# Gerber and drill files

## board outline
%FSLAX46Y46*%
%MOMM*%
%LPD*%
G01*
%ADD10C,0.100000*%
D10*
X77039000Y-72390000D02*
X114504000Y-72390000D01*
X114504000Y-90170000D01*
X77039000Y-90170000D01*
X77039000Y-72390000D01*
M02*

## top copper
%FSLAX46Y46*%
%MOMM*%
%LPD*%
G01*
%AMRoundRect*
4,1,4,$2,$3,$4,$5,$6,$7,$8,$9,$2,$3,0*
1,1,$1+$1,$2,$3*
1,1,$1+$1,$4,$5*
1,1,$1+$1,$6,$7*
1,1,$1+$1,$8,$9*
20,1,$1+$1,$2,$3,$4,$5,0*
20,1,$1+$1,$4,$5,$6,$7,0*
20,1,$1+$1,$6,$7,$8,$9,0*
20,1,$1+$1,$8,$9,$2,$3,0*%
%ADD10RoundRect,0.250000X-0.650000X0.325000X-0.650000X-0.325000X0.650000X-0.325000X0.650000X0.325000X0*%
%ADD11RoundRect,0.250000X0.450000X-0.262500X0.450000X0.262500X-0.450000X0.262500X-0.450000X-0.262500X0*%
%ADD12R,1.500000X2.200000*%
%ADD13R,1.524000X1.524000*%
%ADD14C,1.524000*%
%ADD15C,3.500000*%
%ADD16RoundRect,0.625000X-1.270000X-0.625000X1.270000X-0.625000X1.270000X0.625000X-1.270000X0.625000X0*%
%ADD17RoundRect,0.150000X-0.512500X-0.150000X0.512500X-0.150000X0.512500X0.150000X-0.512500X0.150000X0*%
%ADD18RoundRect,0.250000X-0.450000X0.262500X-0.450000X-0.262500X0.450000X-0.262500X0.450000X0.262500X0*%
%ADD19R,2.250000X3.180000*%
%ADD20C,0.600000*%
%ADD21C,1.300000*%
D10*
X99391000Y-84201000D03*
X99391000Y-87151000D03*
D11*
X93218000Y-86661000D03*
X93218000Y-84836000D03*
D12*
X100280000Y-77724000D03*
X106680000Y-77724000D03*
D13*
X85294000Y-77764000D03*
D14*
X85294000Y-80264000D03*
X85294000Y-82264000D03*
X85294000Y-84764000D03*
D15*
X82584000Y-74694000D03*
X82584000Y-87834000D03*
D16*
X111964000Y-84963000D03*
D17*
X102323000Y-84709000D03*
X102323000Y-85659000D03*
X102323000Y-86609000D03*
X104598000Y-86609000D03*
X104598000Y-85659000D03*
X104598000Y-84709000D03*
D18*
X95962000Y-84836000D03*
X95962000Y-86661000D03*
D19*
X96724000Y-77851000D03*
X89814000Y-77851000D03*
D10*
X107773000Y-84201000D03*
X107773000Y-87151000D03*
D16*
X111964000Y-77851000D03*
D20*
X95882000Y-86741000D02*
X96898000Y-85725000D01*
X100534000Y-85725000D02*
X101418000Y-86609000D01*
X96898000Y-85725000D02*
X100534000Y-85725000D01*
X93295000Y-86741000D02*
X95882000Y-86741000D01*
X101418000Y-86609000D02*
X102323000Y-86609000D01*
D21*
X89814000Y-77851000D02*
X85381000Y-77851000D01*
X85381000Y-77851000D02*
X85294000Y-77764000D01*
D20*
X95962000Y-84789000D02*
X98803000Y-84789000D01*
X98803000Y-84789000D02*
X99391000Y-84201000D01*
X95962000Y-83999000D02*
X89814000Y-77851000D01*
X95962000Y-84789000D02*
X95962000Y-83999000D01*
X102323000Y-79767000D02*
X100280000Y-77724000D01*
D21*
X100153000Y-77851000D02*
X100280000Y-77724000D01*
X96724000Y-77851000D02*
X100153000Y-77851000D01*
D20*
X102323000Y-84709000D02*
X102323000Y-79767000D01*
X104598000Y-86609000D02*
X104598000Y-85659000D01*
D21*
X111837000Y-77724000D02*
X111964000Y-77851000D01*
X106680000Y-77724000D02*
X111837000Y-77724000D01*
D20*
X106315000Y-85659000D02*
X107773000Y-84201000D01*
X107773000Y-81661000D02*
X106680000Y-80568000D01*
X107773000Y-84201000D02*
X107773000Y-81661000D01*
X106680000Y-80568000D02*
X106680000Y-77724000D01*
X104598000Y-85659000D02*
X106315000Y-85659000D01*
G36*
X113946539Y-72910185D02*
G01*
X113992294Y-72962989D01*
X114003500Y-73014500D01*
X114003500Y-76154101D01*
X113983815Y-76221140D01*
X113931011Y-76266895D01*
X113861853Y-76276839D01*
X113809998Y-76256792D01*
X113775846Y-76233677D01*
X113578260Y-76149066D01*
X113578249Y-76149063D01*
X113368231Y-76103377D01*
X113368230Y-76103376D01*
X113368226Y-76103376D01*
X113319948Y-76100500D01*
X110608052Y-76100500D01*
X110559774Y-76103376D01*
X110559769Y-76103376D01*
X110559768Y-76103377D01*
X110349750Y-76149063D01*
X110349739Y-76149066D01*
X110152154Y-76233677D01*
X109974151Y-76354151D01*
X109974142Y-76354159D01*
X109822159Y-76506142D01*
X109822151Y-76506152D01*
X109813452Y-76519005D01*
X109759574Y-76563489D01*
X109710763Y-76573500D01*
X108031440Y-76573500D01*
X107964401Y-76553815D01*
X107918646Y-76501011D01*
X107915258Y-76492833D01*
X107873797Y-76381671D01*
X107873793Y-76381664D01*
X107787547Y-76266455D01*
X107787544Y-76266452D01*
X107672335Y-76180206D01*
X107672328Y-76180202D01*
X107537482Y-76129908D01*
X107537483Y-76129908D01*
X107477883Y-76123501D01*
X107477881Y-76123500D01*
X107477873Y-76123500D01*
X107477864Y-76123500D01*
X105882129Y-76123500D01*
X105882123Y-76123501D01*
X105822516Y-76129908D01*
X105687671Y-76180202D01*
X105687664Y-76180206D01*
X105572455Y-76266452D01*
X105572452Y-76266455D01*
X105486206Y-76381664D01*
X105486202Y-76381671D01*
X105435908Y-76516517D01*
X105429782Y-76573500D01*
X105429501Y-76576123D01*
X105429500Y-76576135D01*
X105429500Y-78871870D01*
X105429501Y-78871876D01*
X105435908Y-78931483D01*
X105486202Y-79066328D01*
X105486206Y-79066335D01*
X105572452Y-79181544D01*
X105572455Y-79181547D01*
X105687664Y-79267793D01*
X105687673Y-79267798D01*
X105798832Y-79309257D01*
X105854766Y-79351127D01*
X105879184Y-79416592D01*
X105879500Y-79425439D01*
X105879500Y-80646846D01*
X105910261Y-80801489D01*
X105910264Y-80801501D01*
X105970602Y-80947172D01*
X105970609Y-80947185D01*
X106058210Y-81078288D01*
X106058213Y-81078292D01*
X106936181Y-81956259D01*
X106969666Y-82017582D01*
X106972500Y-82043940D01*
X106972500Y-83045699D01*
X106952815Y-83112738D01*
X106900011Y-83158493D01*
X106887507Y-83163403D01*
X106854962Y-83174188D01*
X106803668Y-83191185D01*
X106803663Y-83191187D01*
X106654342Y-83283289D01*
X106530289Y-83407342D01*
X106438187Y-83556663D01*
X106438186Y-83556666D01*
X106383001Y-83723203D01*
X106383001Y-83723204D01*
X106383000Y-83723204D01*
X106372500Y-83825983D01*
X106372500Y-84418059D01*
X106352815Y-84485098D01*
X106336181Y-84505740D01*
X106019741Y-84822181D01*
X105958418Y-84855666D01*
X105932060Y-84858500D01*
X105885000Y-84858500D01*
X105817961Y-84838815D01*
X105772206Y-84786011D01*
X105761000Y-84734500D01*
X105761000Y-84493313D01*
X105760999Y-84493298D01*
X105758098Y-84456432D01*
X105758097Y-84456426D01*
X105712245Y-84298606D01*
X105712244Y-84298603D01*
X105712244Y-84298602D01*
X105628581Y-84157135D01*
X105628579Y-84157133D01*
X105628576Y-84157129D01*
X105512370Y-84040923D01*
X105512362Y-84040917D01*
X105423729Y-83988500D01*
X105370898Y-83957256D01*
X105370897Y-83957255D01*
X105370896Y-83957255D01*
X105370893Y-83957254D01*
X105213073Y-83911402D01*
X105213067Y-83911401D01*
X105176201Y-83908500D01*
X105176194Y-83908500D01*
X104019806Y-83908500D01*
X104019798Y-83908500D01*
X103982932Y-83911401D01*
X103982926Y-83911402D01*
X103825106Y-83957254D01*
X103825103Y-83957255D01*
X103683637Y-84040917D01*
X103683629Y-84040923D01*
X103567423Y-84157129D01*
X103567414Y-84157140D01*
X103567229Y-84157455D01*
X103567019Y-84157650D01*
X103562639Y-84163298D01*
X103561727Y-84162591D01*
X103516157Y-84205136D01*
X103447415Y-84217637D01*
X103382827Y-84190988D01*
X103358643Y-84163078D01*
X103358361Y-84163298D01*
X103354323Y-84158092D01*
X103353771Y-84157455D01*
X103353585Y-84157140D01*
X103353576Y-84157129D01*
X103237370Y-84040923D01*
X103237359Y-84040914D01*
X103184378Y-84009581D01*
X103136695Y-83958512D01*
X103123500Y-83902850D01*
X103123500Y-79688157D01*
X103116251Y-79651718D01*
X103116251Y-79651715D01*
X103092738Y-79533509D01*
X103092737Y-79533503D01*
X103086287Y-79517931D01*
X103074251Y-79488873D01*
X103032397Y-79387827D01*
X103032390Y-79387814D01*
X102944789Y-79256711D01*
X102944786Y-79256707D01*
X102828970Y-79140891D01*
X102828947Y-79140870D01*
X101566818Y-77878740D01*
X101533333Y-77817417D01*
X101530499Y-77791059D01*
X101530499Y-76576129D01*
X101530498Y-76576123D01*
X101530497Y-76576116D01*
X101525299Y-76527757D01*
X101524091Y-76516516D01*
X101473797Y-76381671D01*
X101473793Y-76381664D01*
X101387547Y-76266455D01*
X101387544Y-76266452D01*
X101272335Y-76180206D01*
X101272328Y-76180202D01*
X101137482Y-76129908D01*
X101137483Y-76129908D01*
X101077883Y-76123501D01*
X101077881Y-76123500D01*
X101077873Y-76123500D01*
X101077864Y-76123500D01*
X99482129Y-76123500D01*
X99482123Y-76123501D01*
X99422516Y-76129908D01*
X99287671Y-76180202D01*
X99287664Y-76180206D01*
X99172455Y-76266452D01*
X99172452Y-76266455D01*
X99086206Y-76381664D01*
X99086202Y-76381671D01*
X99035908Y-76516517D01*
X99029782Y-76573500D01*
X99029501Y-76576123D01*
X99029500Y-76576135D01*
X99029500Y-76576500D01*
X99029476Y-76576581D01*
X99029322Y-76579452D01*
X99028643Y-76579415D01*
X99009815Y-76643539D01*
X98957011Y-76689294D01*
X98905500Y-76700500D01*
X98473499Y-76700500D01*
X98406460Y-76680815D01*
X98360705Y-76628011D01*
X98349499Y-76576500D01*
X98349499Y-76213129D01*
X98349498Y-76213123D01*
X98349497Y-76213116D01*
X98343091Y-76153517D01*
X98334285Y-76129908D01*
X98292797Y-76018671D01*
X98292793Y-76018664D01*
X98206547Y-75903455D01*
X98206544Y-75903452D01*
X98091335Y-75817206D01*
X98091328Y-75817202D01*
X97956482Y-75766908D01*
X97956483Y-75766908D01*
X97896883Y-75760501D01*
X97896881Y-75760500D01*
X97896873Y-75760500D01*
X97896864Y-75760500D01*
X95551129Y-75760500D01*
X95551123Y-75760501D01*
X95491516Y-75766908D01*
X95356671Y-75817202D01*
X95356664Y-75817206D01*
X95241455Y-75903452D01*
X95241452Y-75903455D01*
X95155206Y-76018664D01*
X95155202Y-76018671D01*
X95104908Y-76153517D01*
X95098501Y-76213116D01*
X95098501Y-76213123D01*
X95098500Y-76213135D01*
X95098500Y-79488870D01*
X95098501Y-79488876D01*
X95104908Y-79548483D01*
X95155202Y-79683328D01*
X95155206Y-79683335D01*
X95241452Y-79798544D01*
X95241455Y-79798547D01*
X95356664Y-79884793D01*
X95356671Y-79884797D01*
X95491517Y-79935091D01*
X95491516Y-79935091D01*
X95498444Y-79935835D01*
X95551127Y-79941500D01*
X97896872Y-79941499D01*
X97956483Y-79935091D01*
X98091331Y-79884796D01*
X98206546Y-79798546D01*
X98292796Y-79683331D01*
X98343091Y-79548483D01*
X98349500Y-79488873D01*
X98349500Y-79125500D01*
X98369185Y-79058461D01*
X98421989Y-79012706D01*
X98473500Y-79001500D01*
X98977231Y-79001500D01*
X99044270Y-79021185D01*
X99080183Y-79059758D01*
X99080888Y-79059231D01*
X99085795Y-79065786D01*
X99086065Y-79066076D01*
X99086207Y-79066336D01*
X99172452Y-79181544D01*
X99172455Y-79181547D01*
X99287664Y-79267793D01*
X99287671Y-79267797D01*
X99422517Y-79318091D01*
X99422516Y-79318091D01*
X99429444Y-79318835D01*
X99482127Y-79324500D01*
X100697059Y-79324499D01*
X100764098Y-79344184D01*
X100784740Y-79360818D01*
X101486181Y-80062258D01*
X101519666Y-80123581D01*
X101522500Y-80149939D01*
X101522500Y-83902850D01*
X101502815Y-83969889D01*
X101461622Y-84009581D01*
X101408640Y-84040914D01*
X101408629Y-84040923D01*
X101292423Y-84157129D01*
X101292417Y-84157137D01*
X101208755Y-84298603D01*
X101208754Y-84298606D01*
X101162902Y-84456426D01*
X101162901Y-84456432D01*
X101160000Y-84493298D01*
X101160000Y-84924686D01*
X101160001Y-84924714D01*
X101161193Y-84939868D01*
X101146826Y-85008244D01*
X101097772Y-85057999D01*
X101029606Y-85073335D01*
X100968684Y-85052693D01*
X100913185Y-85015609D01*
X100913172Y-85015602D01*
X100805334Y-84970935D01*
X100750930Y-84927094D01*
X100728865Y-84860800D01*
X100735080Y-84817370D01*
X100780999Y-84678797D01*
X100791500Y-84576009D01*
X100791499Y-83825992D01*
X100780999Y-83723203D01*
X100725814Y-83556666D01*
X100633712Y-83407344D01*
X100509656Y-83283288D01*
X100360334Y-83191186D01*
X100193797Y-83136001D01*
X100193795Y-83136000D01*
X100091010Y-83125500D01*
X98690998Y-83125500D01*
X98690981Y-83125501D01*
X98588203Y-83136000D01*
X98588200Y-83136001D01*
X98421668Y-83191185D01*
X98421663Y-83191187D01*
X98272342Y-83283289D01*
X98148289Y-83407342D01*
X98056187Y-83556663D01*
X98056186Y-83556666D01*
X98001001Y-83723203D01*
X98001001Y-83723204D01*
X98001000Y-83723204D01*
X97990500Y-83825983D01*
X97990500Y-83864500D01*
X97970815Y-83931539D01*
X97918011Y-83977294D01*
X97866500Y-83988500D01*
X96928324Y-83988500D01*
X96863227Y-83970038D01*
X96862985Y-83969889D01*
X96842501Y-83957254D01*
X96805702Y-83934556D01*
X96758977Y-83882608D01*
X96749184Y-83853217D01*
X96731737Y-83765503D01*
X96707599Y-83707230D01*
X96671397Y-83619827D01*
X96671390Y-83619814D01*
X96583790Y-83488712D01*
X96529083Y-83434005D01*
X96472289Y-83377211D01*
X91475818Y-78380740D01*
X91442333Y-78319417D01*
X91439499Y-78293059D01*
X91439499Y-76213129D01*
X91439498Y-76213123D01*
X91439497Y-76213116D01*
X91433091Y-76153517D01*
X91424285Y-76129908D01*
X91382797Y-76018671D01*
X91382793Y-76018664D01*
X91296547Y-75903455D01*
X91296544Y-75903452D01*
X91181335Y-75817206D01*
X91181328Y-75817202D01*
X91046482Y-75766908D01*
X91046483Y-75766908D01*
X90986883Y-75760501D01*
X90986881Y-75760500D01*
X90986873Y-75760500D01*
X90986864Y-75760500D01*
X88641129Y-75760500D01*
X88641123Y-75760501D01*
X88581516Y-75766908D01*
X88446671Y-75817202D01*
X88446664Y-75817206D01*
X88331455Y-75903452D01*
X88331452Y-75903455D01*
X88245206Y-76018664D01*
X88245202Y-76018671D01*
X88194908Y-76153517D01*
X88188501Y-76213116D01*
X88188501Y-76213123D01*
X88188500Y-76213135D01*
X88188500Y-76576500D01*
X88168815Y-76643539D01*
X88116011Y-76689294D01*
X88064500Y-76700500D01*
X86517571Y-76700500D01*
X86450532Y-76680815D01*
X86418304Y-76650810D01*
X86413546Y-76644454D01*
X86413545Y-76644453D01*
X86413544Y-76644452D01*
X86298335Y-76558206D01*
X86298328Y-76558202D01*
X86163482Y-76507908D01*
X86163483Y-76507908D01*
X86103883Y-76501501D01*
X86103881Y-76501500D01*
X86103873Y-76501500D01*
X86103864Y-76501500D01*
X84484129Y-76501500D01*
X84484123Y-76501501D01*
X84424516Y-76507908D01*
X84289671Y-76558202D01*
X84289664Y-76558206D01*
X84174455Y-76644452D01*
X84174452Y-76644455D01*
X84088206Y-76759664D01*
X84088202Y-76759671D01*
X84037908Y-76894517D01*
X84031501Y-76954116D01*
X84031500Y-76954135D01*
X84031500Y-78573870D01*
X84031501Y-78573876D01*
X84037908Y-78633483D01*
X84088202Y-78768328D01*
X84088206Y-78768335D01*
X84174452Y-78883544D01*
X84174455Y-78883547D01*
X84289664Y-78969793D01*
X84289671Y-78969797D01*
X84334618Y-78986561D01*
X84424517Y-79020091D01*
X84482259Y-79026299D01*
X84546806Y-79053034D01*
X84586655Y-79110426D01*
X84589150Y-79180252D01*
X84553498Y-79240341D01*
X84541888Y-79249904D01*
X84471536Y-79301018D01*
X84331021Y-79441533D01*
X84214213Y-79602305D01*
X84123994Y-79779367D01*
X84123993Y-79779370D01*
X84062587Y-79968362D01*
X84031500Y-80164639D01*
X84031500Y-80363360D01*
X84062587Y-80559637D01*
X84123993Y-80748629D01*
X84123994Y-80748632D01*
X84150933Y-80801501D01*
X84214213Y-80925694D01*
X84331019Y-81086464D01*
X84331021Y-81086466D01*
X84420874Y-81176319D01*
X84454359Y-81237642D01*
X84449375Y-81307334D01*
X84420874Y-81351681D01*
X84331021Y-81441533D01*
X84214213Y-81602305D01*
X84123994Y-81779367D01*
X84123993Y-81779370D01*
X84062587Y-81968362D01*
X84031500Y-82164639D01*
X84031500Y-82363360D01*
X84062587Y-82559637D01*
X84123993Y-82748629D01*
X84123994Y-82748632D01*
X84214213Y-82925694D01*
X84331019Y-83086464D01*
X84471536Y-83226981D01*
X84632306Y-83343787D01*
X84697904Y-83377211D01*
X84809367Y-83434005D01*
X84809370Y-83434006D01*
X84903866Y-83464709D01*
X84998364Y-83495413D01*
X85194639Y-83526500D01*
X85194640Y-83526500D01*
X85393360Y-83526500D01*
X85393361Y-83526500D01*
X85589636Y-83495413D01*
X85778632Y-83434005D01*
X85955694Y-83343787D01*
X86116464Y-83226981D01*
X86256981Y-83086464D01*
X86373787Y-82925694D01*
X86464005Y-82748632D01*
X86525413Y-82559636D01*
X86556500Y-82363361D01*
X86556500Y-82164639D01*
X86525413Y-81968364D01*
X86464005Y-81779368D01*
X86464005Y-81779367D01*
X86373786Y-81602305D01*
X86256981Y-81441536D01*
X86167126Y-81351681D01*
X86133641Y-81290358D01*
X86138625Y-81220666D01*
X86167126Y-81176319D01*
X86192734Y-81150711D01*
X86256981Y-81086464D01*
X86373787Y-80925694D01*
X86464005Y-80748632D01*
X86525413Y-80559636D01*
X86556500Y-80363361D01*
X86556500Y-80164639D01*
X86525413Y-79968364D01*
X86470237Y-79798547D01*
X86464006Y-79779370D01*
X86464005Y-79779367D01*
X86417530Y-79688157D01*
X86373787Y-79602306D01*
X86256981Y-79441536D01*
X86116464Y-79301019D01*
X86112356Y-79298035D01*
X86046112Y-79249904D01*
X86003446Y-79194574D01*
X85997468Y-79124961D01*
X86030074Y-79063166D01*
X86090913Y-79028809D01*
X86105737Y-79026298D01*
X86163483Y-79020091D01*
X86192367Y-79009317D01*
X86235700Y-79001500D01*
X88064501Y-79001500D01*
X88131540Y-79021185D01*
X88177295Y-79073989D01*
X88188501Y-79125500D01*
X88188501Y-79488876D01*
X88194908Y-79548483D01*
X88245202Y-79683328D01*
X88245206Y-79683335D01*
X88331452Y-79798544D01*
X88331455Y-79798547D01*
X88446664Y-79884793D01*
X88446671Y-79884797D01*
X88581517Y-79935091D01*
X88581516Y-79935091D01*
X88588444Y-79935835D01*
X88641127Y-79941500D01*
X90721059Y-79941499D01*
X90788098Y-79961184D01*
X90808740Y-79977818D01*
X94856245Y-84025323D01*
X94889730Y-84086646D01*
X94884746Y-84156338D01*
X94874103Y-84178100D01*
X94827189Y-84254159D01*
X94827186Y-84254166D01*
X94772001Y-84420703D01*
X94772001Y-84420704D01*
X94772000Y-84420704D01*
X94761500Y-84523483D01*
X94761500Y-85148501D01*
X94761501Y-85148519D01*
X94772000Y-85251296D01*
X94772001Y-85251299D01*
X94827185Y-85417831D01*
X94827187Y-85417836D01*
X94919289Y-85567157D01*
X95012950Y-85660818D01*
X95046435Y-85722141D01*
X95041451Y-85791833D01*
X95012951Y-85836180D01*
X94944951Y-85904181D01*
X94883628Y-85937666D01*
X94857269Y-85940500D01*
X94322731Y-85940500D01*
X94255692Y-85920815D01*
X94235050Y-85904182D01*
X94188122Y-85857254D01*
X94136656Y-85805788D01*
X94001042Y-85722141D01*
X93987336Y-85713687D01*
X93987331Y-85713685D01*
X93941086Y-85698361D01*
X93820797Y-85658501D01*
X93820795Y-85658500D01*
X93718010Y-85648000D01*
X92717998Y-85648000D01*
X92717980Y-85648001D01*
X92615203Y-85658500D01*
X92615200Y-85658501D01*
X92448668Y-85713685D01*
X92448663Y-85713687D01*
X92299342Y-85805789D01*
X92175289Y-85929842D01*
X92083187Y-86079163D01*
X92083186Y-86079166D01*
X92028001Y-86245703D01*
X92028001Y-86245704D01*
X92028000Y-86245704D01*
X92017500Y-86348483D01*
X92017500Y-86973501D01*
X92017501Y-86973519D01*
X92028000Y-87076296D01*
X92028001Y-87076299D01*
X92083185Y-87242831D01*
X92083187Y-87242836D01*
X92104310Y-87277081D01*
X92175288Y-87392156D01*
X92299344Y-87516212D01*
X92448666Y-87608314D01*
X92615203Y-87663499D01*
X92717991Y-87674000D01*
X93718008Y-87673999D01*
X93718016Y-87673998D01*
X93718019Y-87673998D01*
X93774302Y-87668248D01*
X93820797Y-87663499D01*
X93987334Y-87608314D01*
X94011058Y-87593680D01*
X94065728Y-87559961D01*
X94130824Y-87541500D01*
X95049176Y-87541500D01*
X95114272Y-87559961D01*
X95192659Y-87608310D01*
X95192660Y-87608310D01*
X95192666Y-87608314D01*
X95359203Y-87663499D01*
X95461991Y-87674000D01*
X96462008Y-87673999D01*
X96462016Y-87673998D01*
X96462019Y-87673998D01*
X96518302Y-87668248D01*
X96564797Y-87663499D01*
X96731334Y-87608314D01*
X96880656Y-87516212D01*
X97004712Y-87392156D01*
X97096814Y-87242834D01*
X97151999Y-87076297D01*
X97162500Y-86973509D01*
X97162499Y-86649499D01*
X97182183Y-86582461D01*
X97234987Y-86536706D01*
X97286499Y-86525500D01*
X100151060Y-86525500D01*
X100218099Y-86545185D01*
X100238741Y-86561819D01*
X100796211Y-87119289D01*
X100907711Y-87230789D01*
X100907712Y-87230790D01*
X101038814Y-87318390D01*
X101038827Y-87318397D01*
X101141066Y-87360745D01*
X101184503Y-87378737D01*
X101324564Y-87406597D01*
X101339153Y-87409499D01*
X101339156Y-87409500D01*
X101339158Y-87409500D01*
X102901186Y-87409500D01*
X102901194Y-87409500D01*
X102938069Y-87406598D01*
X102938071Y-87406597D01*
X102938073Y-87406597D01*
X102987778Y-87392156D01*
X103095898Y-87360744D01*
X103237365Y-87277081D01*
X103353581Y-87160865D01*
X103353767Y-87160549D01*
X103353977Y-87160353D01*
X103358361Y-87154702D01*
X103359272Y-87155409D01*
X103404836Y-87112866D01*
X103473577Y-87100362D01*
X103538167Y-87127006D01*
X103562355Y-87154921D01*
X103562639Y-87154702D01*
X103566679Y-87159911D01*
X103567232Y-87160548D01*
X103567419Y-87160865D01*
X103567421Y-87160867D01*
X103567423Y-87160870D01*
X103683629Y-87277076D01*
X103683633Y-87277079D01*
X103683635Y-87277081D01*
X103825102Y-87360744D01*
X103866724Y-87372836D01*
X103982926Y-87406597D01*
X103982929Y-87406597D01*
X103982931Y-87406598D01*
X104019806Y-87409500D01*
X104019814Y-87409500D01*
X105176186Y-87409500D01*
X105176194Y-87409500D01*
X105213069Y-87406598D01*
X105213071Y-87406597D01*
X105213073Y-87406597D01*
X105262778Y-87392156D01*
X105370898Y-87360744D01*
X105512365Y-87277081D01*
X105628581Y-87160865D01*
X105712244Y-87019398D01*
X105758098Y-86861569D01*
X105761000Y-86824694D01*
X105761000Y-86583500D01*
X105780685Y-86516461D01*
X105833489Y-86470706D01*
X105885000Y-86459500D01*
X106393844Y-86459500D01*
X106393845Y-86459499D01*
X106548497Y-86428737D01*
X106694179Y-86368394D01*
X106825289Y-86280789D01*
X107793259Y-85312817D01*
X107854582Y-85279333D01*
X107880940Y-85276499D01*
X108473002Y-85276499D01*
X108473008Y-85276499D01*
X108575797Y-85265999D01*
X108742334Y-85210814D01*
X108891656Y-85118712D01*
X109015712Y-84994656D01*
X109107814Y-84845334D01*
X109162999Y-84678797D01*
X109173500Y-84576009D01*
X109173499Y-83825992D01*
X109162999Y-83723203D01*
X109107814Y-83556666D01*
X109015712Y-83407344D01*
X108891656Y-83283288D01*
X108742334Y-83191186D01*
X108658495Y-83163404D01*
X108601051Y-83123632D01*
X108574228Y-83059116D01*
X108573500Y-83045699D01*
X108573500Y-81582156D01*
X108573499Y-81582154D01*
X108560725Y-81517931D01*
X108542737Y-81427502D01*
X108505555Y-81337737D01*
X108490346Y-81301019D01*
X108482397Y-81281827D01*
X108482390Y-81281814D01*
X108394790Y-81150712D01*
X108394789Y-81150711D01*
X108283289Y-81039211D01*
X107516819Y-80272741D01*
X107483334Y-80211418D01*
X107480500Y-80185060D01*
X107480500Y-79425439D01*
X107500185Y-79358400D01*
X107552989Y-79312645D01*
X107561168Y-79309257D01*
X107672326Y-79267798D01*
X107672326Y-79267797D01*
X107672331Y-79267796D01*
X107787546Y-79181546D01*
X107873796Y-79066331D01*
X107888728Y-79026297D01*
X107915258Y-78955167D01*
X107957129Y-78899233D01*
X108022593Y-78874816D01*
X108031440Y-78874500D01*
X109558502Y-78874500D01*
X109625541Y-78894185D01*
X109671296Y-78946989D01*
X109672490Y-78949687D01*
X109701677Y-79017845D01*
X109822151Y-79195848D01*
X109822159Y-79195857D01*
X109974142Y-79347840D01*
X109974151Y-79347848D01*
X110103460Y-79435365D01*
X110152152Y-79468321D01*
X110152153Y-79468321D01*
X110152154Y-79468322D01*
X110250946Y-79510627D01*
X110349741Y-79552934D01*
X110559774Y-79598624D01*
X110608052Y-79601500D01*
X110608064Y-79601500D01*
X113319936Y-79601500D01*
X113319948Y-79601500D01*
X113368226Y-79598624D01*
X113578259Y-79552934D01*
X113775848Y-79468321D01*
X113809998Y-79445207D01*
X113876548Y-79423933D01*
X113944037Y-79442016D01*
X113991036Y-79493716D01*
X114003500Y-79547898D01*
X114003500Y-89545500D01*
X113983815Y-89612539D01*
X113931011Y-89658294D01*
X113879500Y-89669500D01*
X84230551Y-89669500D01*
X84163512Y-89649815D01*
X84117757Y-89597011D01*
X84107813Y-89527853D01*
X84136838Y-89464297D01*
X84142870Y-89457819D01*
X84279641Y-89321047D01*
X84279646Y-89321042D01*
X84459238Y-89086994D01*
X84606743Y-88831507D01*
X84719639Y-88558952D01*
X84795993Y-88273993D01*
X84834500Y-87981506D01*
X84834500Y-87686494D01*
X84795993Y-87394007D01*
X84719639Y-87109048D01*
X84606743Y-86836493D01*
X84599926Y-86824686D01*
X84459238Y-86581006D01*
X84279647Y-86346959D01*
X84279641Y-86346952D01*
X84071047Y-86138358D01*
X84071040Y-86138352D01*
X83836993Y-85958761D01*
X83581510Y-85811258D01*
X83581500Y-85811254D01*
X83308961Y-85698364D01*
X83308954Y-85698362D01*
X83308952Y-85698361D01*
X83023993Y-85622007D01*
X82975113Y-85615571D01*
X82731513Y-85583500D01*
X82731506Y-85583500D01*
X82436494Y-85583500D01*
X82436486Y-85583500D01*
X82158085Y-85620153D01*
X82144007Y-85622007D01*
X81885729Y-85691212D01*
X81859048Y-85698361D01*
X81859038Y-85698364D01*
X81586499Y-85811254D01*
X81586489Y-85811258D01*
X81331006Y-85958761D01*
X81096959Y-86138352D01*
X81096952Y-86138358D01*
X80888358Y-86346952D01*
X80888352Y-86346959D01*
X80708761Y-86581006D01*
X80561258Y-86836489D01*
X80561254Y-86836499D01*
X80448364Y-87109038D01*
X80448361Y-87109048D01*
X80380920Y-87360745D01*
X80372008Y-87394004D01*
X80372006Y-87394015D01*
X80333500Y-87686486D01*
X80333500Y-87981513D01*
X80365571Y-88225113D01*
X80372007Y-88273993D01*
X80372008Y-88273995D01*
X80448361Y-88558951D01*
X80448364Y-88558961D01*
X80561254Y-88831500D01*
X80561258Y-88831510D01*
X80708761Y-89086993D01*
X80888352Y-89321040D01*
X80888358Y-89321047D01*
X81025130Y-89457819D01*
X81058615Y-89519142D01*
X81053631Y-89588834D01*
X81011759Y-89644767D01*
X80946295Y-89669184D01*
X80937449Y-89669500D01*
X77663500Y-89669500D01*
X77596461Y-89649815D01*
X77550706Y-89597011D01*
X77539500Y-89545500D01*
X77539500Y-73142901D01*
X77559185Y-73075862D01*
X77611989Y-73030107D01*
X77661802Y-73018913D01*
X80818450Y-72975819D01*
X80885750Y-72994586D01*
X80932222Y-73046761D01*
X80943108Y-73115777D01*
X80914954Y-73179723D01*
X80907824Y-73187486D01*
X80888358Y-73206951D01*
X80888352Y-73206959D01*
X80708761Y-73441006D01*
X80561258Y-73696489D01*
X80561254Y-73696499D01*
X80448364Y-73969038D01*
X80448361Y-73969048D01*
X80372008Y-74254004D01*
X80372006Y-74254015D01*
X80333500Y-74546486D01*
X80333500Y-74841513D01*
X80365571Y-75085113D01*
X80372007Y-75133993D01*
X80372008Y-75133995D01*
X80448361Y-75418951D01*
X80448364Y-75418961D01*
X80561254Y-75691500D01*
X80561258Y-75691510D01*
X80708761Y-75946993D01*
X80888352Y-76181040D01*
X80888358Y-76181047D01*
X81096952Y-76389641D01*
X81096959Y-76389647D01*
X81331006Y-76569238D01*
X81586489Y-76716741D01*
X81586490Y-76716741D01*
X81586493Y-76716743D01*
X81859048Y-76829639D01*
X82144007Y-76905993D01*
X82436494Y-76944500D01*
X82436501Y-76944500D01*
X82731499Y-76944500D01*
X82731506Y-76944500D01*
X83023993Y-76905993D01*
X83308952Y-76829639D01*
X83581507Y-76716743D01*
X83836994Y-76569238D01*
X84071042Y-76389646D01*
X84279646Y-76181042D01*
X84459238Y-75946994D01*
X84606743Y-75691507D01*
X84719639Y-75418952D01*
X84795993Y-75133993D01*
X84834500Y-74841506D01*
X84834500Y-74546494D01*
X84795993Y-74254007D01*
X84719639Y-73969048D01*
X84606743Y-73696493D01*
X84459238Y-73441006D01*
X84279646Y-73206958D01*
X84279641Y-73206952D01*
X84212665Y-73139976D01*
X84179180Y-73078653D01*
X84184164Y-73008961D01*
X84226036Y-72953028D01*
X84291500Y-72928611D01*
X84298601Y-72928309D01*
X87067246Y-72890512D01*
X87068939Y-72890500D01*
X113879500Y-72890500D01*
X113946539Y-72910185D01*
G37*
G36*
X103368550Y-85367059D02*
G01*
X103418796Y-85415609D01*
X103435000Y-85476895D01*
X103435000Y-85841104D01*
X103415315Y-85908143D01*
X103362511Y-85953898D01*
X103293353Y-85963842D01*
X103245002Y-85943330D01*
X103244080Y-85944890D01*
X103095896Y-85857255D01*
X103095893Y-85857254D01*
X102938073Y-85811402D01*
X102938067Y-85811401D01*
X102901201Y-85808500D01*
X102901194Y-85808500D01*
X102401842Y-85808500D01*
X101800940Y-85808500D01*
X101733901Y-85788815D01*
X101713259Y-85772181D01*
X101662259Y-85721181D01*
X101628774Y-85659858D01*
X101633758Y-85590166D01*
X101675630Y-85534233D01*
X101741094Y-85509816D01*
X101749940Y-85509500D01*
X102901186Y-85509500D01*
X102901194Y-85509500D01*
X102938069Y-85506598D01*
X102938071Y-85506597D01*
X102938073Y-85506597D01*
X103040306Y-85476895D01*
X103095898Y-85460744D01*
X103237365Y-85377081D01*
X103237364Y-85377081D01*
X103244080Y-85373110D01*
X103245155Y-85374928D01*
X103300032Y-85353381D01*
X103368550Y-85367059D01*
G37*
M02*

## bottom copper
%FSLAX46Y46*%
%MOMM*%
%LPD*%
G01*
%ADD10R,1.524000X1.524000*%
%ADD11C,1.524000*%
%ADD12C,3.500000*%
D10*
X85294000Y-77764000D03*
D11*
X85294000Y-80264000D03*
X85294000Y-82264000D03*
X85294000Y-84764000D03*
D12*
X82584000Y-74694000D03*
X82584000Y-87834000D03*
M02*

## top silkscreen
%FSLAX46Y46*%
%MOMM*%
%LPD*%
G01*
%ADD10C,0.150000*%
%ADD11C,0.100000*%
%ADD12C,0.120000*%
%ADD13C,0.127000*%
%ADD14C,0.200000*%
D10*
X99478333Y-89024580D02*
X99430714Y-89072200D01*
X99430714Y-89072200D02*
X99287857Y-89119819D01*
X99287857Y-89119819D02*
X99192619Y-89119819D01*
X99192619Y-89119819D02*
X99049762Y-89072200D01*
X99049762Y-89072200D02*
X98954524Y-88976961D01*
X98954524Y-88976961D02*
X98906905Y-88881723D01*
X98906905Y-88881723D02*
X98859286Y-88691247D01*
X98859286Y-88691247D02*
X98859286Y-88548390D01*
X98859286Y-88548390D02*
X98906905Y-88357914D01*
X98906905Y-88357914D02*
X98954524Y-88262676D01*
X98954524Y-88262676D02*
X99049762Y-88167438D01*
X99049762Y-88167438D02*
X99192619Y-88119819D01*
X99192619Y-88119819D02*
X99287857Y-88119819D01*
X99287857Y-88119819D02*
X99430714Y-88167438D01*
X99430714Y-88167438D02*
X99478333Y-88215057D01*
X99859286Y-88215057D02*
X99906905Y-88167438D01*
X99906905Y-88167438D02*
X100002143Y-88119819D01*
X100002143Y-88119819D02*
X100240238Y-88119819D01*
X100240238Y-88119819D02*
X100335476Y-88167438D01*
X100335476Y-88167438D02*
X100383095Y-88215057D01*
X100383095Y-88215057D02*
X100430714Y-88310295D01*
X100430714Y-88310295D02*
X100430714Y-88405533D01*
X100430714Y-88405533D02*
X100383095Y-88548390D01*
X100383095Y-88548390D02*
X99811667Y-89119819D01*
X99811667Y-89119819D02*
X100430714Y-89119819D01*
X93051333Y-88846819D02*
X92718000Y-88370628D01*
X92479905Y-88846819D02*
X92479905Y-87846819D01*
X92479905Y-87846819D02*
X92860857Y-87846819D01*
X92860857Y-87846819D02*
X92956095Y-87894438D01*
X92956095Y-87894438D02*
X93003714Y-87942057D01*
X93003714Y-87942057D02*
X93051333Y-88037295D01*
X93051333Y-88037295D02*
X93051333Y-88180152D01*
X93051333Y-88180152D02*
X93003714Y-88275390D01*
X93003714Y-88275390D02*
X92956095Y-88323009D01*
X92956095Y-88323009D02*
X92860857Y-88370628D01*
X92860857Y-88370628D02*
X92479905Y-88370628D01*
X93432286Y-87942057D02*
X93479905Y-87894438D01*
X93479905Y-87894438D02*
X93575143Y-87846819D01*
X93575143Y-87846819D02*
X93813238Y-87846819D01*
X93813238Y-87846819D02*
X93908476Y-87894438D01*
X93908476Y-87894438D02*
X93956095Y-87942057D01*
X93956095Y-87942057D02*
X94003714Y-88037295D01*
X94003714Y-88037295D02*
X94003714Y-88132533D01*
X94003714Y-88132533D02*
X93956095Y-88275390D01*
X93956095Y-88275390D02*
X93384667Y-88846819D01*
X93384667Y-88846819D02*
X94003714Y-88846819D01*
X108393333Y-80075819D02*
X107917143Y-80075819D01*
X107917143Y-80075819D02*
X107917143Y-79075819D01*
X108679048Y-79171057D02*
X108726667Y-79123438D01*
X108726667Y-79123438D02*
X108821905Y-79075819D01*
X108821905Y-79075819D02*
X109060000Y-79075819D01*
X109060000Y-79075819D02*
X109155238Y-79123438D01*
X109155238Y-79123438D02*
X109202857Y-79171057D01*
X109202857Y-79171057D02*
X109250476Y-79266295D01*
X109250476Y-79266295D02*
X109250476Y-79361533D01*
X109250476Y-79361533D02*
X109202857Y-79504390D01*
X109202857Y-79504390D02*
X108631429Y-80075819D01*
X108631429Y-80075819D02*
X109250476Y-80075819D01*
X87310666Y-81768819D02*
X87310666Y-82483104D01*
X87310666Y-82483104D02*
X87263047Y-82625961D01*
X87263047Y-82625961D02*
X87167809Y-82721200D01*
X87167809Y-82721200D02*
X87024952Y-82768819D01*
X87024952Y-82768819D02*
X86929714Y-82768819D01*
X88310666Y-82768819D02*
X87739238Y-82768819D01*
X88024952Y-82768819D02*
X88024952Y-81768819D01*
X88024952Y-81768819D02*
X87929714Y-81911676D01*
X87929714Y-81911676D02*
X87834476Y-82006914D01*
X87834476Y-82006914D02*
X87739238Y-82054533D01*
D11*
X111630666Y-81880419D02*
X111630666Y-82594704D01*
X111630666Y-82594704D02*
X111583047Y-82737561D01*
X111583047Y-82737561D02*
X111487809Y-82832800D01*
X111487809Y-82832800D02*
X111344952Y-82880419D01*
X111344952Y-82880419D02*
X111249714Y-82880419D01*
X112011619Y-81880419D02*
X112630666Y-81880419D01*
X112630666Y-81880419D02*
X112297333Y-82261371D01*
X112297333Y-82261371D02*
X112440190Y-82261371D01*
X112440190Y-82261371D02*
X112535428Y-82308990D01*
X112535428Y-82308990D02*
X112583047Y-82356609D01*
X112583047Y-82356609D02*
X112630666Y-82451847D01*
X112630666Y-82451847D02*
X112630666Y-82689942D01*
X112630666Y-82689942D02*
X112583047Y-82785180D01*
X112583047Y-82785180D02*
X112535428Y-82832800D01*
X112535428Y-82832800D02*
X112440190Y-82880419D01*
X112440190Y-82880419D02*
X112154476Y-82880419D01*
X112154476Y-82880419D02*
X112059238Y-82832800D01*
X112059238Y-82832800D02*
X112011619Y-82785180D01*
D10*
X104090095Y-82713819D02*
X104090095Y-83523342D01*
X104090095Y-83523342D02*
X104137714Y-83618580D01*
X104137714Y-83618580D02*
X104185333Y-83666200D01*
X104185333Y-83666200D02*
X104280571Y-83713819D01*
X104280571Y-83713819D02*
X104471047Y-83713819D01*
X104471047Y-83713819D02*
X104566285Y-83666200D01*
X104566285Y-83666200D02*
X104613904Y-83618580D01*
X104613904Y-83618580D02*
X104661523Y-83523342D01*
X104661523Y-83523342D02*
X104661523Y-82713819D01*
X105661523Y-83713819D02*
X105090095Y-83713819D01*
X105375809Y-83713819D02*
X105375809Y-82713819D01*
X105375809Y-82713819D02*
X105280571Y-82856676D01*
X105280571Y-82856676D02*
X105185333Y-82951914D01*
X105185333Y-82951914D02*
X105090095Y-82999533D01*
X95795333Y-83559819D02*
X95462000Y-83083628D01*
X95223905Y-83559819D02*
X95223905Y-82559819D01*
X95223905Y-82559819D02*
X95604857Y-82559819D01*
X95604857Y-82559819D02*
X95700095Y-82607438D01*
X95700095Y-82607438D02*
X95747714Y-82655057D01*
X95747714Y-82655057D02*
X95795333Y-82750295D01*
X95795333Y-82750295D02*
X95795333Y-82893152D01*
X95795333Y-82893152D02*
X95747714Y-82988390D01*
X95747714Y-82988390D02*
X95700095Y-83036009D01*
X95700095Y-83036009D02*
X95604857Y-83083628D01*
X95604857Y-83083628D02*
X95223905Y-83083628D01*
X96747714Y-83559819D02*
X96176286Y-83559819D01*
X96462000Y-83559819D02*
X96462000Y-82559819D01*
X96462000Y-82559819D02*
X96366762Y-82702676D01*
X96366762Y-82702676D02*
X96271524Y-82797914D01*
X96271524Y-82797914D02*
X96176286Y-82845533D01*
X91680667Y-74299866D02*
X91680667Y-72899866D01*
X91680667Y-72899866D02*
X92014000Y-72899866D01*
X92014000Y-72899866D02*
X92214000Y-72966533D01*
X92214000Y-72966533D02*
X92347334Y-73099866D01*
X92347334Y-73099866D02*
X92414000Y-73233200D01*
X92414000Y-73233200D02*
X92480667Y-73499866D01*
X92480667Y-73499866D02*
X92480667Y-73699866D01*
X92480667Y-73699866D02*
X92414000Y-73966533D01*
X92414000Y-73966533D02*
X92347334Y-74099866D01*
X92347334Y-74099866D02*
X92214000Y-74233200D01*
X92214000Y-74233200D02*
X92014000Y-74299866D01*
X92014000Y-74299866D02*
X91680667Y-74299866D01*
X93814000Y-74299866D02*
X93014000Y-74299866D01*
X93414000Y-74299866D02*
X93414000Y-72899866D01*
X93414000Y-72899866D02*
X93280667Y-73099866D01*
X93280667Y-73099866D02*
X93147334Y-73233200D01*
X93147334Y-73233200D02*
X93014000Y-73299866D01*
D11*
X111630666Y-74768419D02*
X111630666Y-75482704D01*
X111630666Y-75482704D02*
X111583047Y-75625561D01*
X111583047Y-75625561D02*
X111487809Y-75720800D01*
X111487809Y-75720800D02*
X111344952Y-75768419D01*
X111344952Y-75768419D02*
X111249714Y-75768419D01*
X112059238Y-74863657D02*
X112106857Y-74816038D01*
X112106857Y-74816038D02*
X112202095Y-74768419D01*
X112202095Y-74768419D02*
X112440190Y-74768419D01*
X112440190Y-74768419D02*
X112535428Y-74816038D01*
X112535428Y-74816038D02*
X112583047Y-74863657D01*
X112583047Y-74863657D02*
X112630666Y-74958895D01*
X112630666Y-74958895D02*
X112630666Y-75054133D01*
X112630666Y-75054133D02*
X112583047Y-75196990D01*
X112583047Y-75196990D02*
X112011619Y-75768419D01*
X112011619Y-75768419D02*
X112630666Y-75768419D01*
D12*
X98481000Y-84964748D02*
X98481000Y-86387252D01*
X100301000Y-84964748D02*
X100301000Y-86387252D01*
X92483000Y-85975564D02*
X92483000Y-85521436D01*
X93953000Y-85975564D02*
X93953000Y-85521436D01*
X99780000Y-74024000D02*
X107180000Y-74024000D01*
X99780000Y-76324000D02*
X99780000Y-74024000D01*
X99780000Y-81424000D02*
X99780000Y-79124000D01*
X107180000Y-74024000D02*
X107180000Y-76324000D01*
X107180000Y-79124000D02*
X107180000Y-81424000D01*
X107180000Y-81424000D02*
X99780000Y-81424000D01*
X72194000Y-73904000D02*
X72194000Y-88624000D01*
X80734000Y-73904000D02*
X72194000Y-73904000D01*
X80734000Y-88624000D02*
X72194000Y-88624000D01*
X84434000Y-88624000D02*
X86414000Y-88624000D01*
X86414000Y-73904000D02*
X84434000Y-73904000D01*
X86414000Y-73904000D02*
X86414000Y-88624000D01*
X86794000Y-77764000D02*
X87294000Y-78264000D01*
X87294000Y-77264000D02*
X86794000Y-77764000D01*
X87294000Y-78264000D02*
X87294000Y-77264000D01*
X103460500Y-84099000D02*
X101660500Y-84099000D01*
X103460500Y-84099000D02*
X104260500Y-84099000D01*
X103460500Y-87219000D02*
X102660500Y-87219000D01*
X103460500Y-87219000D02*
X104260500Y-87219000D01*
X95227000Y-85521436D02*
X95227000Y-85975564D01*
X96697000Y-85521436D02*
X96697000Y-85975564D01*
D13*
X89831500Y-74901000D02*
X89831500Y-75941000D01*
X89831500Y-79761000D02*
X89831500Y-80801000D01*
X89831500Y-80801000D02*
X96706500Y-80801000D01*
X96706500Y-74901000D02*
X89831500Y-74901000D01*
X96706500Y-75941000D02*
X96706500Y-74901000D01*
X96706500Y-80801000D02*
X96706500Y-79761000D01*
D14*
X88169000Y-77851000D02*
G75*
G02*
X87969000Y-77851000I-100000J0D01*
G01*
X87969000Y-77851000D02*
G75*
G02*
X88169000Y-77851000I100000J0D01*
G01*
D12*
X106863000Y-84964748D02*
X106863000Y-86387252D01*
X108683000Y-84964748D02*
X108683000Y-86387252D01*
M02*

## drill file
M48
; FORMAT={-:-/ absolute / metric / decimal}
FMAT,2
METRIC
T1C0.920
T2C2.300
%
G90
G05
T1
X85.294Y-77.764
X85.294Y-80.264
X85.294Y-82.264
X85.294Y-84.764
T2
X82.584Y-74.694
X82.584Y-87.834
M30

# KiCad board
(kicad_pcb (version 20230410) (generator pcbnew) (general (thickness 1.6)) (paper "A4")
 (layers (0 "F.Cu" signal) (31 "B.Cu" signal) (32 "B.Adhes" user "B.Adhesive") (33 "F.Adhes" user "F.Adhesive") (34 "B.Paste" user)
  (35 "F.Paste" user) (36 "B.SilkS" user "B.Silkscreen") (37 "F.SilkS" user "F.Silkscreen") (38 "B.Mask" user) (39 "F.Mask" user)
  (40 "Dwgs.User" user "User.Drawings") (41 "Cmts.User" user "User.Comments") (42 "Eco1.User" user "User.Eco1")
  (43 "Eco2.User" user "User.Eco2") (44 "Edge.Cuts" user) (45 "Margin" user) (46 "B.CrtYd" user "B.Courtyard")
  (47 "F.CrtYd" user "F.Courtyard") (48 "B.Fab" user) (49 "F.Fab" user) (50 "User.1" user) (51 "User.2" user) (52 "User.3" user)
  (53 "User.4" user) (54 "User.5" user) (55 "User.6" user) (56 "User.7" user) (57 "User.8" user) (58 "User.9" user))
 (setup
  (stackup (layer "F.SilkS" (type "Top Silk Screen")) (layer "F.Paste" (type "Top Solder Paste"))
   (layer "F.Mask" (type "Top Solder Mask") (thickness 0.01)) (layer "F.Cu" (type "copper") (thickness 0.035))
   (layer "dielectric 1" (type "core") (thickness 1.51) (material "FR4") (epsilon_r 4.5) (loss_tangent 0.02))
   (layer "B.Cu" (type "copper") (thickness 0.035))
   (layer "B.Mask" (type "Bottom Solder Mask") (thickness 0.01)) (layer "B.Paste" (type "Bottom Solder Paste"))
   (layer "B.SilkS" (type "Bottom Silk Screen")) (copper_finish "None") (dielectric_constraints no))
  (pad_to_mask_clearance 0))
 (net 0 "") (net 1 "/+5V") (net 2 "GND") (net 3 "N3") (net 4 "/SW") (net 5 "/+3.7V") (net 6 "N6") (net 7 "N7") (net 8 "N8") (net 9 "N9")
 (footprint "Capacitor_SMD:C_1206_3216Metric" (layer "F.Cu") (at 99.391 85.676 -90)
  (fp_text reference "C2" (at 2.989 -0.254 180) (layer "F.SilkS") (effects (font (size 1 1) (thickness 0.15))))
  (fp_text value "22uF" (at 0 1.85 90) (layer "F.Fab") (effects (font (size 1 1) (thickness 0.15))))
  (fp_line (start -0.711252 0.91) (end 0.711252 0.91) (stroke (width 0.12) (type solid)) (layer "F.SilkS"))
  (fp_line (start -0.711252 -0.91) (end 0.711252 -0.91) (stroke (width 0.12) (type solid)) (layer "F.SilkS"))
  (pad "1" smd roundrect (at -1.475 0 270) (size 1.15 1.8) (layers "F.Cu" "F.Paste" "F.Mask") (roundrect_rratio 0.217391) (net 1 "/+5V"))
  (pad "2" smd roundrect (at 1.475 0 270) (size 1.15 1.8) (layers "F.Cu" "F.Paste" "F.Mask") (roundrect_rratio 0.217391) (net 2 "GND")))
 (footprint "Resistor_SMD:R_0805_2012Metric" (layer "F.Cu") (at 93.218 85.7485 90)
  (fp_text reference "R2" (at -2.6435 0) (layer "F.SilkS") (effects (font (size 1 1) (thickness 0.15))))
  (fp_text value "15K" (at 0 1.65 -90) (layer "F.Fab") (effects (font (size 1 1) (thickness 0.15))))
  (fp_line (start -0.227064 -0.735) (end 0.227064 -0.735) (stroke (width 0.12) (type solid)) (layer "F.SilkS"))
  (fp_line (start -0.227064 0.735) (end 0.227064 0.735) (stroke (width 0.12) (type solid)) (layer "F.SilkS"))
  (pad "1" smd roundrect (at -0.9125 0 90) (size 1.025 1.4) (layers "F.Cu" "F.Paste" "F.Mask") (roundrect_rratio 0.243902) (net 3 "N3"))
  (pad "2" smd roundrect (at 0.9125 0 90) (size 1.025 1.4) (layers "F.Cu" "F.Paste" "F.Mask") (roundrect_rratio 0.243902) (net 2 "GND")))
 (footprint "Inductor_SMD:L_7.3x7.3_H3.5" (layer "F.Cu") (at 103.48 77.724)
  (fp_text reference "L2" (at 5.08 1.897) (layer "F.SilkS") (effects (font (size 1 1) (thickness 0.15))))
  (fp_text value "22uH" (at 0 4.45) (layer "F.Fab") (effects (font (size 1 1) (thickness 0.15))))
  (fp_line (start -3.7 -3.7) (end 3.7 -3.7) (stroke (width 0.12) (type solid)) (layer "F.SilkS"))
  (fp_line (start -3.7 -1.4) (end -3.7 -3.7) (stroke (width 0.12) (type solid)) (layer "F.SilkS"))
  (fp_line (start -3.7 3.7) (end -3.7 1.4) (stroke (width 0.12) (type solid)) (layer "F.SilkS"))
  (fp_line (start 3.7 -3.7) (end 3.7 -1.4) (stroke (width 0.12) (type solid)) (layer "F.SilkS"))
  (fp_line (start 3.7 1.4) (end 3.7 3.7) (stroke (width 0.12) (type solid)) (layer "F.SilkS"))
  (fp_line (start 3.7 3.7) (end -3.7 3.7) (stroke (width 0.12) (type solid)) (layer "F.SilkS"))
  (pad "1" smd rect (at -3.2 0) (size 1.5 2.2) (layers "F.Cu" "F.Paste" "F.Mask") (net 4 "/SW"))
  (pad "2" smd rect (at 3.2 0) (size 1.5 2.2) (layers "F.Cu" "F.Paste" "F.Mask") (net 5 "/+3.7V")))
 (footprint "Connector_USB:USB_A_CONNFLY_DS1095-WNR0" (layer "F.Cu") (at 85.294 77.764 -90)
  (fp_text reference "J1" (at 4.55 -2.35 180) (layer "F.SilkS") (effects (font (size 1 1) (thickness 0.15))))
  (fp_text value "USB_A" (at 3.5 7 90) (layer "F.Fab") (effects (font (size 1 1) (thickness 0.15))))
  (fp_line (start -3.86 13.1) (end 10.86 13.1) (stroke (width 0.12) (type solid)) (layer "F.SilkS"))
  (fp_line (start -3.86 4.56) (end -3.86 13.1) (stroke (width 0.12) (type solid)) (layer "F.SilkS"))
  (fp_line (start 10.86 4.56) (end 10.86 13.1) (stroke (width 0.12) (type solid)) (layer "F.SilkS"))
  (fp_line (start 10.86 0.86) (end 10.86 -1.12) (stroke (width 0.12) (type solid)) (layer "F.SilkS"))
  (fp_line (start -3.86 -1.12) (end -3.86 0.86) (stroke (width 0.12) (type solid)) (layer "F.SilkS"))
  (fp_line (start -3.86 -1.12) (end 10.86 -1.12) (stroke (width 0.12) (type solid)) (layer "F.SilkS"))
  (fp_line (start 0 -1.5) (end 0.5 -2) (stroke (width 0.12) (type solid)) (layer "F.SilkS"))
  (fp_line (start -0.5 -2) (end 0 -1.5) (stroke (width 0.12) (type solid)) (layer "F.SilkS"))
  (fp_line (start 0.5 -2) (end -0.5 -2) (stroke (width 0.12) (type solid)) (layer "F.SilkS"))
  (pad "1" thru_hole rect (at 0 0 270) (size 1.524 1.524) (drill 0.92) (layers "*.Cu" "*.Mask") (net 1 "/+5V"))
  (pad "2" thru_hole circle (at 2.5 0 270) (size 1.524 1.524) (drill 0.92) (layers "*.Cu" "*.Mask") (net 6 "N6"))
  (pad "3" thru_hole circle (at 4.5 0 270) (size 1.524 1.524) (drill 0.92) (layers "*.Cu" "*.Mask") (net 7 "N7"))
  (pad "4" thru_hole circle (at 7 0 270) (size 1.524 1.524) (drill 0.92) (layers "*.Cu" "*.Mask") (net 2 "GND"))
  (pad "5" thru_hole circle (at -3.07 2.71 270) (size 3.5 3.5) (drill 2.3) (layers "*.Cu" "*.Mask") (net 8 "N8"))
  (pad "5" thru_hole circle (at 10.07 2.71 270) (size 3.5 3.5) (drill 2.3) (layers "*.Cu" "*.Mask") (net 8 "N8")))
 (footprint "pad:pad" (layer "F.Cu") (at 111.964 84.963)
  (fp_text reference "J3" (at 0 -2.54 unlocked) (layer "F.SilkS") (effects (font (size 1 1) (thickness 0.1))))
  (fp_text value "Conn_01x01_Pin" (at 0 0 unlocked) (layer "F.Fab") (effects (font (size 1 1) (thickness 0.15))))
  (pad "1" smd roundrect (at 0 0) (size 3.79 2.5) (layers "F.Cu" "F.Paste" "F.Mask") (roundrect_rratio 0.25) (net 2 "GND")
   (thermal_bridge_angle 45)))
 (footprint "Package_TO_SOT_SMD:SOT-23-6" (layer "F.Cu") (at 103.4605 85.659)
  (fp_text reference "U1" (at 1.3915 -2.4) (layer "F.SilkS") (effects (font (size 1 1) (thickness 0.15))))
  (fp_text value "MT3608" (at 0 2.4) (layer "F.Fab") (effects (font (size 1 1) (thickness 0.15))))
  (fp_line (start 0 -1.56) (end -1.8 -1.56) (stroke (width 0.12) (type solid)) (layer "F.SilkS"))
  (fp_line (start 0 -1.56) (end 0.8 -1.56) (stroke (width 0.12) (type solid)) (layer "F.SilkS"))
  (fp_line (start 0 1.56) (end -0.8 1.56) (stroke (width 0.12) (type solid)) (layer "F.SilkS"))
  (fp_line (start 0 1.56) (end 0.8 1.56) (stroke (width 0.12) (type solid)) (layer "F.SilkS"))
  (pad "1" smd roundrect (at -1.1375 -0.95) (size 1.325 0.6) (layers "F.Cu" "F.Paste" "F.Mask") (roundrect_rratio 0.25) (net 4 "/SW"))
  (pad "2" smd roundrect (at -1.1375 0) (size 1.325 0.6) (layers "F.Cu" "F.Paste" "F.Mask") (roundrect_rratio 0.25) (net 2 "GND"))
  (pad "3" smd roundrect (at -1.1375 0.95) (size 1.325 0.6) (layers "F.Cu" "F.Paste" "F.Mask") (roundrect_rratio 0.25) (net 3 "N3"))
  (pad "4" smd roundrect (at 1.1375 0.95) (size 1.325 0.6) (layers "F.Cu" "F.Paste" "F.Mask") (roundrect_rratio 0.25) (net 5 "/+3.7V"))
  (pad "5" smd roundrect (at 1.1375 0) (size 1.325 0.6) (layers "F.Cu" "F.Paste" "F.Mask") (roundrect_rratio 0.25) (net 5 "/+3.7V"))
  (pad "6" smd roundrect (at 1.1375 -0.95) (size 1.325 0.6) (layers "F.Cu" "F.Paste" "F.Mask") (roundrect_rratio 0.25) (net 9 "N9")))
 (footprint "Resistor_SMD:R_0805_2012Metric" (layer "F.Cu") (at 95.962 85.7485 -90)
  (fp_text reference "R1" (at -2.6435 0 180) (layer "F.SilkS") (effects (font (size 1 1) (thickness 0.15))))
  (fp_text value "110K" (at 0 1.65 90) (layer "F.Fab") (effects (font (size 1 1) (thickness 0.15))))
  (fp_line (start -0.227064 0.735) (end 0.227064 0.735) (stroke (width 0.12) (type solid)) (layer "F.SilkS"))
  (fp_line (start -0.227064 -0.735) (end 0.227064 -0.735) (stroke (width 0.12) (type solid)) (layer "F.SilkS"))
  (pad "1" smd roundrect (at -0.9125 0 270) (size 1.025 1.4) (layers "F.Cu" "F.Paste" "F.Mask") (roundrect_rratio 0.243902) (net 1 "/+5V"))
  (pad "2" smd roundrect (at 0.9125 0 270) (size 1.025 1.4) (layers "F.Cu" "F.Paste" "F.Mask") (roundrect_rratio 0.243902) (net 3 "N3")))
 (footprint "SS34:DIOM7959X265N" (layer "F.Cu") (at 93.269 77.851)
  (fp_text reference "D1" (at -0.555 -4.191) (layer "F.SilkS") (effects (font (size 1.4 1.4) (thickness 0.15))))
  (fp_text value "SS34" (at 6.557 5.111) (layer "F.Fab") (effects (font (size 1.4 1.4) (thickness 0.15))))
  (fp_line (start -3.4375 -2.95) (end -3.4375 -1.91) (stroke (width 0.127) (type solid)) (layer "F.SilkS"))
  (fp_line (start -3.4375 1.91) (end -3.4375 2.95) (stroke (width 0.127) (type solid)) (layer "F.SilkS"))
  (fp_line (start -3.4375 2.95) (end 3.4375 2.95) (stroke (width 0.127) (type solid)) (layer "F.SilkS"))
  (fp_line (start 3.4375 -2.95) (end -3.4375 -2.95) (stroke (width 0.127) (type solid)) (layer "F.SilkS"))
  (fp_line (start 3.4375 -1.91) (end 3.4375 -2.95) (stroke (width 0.127) (type solid)) (layer "F.SilkS"))
  (fp_line (start 3.4375 2.95) (end 3.4375 1.91) (stroke (width 0.127) (type solid)) (layer "F.SilkS"))
  (fp_circle (center -5.2 0) (end -5.1 0) (stroke (width 0.2) (type solid)) (fill none) (layer "F.SilkS"))
  (pad "A" smd rect (at 3.455 0 180) (size 2.25 3.18) (layers "F.Cu" "F.Paste" "F.Mask") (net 4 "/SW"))
  (pad "C" smd rect (at -3.455 0) (size 2.25 3.18) (layers "F.Cu" "F.Paste" "F.Mask") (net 1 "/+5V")))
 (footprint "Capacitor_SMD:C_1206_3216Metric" (layer "F.Cu") (at 107.773 85.676 -90)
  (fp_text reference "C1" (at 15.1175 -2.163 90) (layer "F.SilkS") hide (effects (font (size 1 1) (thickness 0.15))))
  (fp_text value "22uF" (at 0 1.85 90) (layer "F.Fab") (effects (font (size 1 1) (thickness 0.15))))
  (fp_line (start -0.711252 0.91) (end 0.711252 0.91) (stroke (width 0.12) (type solid)) (layer "F.SilkS"))
  (fp_line (start -0.711252 -0.91) (end 0.711252 -0.91) (stroke (width 0.12) (type solid)) (layer "F.SilkS"))
  (pad "1" smd roundrect (at -1.475 0 270) (size 1.15 1.8) (layers "F.Cu" "F.Paste" "F.Mask") (roundrect_rratio 0.217391) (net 5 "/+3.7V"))
  (pad "2" smd roundrect (at 1.475 0 270) (size 1.15 1.8) (layers "F.Cu" "F.Paste" "F.Mask") (roundrect_rratio 0.217391) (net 2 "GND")))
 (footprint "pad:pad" (layer "F.Cu") (at 111.964 77.851)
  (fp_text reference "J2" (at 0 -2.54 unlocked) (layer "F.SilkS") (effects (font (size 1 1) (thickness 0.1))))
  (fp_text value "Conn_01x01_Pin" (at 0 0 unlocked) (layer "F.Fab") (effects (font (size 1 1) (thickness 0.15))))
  (pad "1" smd roundrect (at 0 0) (size 3.79 2.5) (layers "F.Cu" "F.Paste" "F.Mask") (roundrect_rratio 0.25) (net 5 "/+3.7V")
   (thermal_bridge_angle 45)))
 (gr_rect (start 77.039 72.39) (end 114.504 90.17) (stroke (width 0.1) (type default)) (fill none) (layer "Edge.Cuts"))
 (segment (start 95.882 86.741) (end 96.898 85.725) (width 0.6) (layer "F.Cu") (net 3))
 (segment (start 100.534 85.725) (end 101.418 86.609) (width 0.6) (layer "F.Cu") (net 3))
 (segment (start 96.898 85.725) (end 100.534 85.725) (width 0.6) (layer "F.Cu") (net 3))
 (segment (start 93.295 86.741) (end 95.882 86.741) (width 0.6) (layer "F.Cu") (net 3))
 (segment (start 101.418 86.609) (end 102.323 86.609) (width 0.6) (layer "F.Cu") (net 3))
 (segment (start 89.814 77.851) (end 85.381 77.851) (width 1.3) (layer "F.Cu") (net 1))
 (segment (start 85.381 77.851) (end 85.294 77.764) (width 1.3) (layer "F.Cu") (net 1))
 (segment (start 95.962 84.789) (end 98.803 84.789) (width 0.6) (layer "F.Cu") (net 1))
 (segment (start 98.803 84.789) (end 99.391 84.201) (width 0.6) (layer "F.Cu") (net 1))
 (segment (start 95.962 83.999) (end 89.814 77.851) (width 0.6) (layer "F.Cu") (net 1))
 (segment (start 95.962 84.789) (end 95.962 83.999) (width 0.6) (layer "F.Cu") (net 1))
 (segment (start 102.323 79.767) (end 100.28 77.724) (width 0.6) (layer "F.Cu") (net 4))
 (segment (start 100.153 77.851) (end 100.28 77.724) (width 1.3) (layer "F.Cu") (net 4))
 (segment (start 96.724 77.851) (end 100.153 77.851) (width 1.3) (layer "F.Cu") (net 4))
 (segment (start 102.323 84.709) (end 102.323 79.767) (width 0.6) (layer "F.Cu") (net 4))
 (segment (start 104.598 86.609) (end 104.598 85.659) (width 0.6) (layer "F.Cu") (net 5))
 (segment (start 111.837 77.724) (end 111.964 77.851) (width 1.3) (layer "F.Cu") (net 5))
 (segment (start 106.68 77.724) (end 111.837 77.724) (width 1.3) (layer "F.Cu") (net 5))
 (segment (start 106.315 85.659) (end 107.773 84.201) (width 0.6) (layer "F.Cu") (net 5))
 (segment (start 107.773 81.661) (end 106.68 80.568) (width 0.6) (layer "F.Cu") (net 5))
 (segment (start 107.773 84.201) (end 107.773 81.661) (width 0.6) (layer "F.Cu") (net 5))
 (segment (start 106.68 80.568) (end 106.68 77.724) (width 0.6) (layer "F.Cu") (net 5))
 (segment (start 104.598 85.659) (end 106.315 85.659) (width 0.6) (layer "F.Cu") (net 5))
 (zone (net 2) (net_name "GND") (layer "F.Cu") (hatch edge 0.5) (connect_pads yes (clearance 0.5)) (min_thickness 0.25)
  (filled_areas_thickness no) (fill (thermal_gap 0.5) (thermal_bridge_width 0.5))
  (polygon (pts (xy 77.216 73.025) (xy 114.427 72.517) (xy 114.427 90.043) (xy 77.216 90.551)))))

